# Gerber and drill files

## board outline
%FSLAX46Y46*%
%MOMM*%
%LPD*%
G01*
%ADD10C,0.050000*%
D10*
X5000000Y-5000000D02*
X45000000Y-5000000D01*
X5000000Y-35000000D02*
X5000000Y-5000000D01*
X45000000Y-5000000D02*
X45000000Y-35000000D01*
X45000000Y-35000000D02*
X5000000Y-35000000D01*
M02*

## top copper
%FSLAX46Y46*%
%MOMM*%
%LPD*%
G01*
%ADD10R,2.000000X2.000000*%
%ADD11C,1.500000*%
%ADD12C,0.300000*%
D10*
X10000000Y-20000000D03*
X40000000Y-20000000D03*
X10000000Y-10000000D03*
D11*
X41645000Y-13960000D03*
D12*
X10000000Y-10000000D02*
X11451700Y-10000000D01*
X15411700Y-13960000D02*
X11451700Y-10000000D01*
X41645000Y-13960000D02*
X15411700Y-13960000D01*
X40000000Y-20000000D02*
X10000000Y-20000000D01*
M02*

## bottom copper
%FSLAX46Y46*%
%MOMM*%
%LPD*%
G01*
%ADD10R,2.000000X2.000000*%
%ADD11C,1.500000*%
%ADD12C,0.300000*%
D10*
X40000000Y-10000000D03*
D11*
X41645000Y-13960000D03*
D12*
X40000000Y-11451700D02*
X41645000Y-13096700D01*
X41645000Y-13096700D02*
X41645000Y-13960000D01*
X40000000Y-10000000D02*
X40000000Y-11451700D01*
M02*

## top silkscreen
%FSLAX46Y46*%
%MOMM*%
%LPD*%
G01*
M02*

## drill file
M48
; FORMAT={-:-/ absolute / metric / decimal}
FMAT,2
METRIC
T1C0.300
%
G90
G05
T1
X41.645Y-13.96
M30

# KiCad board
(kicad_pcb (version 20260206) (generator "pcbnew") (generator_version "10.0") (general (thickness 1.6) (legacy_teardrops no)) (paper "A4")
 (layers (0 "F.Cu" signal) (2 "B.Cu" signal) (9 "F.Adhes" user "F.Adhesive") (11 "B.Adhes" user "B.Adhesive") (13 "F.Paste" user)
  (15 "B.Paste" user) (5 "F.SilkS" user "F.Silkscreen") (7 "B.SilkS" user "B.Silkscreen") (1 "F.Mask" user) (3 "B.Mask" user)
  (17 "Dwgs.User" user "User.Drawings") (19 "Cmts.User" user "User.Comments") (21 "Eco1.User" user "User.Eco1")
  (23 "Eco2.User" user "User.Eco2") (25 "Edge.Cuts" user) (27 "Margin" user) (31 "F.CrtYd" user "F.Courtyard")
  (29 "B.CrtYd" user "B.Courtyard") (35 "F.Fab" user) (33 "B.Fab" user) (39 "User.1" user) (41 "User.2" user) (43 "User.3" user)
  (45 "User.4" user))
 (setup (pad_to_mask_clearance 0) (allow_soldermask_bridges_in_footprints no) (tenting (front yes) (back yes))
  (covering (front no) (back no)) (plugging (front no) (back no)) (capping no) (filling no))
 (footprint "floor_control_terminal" (layer "F.Cu") (at 10 20)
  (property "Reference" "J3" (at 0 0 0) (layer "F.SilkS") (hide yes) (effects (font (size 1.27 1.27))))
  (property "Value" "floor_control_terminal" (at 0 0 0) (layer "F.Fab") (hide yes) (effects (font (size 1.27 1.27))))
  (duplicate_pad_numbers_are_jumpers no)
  (pad "1" smd rect (at 0 0) (size 2 2) (layers "F.Cu" "F.Mask" "F.Paste") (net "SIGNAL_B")))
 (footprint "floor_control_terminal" (layer "F.Cu") (at 40 20)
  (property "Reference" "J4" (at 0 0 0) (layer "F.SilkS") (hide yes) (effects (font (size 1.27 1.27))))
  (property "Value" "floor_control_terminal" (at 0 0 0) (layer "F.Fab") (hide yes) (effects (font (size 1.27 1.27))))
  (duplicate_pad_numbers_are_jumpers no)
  (pad "1" smd rect (at 0 0) (size 2 2) (layers "F.Cu" "F.Mask" "F.Paste") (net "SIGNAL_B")))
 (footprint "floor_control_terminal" (layer "F.Cu") (at 10 10)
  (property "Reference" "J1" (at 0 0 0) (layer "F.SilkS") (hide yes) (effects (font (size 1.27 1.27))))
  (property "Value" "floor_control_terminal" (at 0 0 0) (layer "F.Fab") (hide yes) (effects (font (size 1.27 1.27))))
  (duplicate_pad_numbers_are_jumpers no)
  (pad "1" smd rect (at 0 0) (size 2 2) (layers "F.Cu" "F.Mask" "F.Paste") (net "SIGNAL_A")))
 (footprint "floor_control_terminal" (layer "B.Cu") (at 40 10)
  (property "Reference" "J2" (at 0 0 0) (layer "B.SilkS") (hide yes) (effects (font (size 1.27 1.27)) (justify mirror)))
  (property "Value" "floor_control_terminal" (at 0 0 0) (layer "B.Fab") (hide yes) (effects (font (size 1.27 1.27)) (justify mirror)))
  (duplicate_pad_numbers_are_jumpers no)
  (pad "1" smd rect (at 0 0) (size 2 2) (layers "B.Cu" "B.Mask" "B.Paste") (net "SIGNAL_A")))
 (gr_line (start 5 5) (end 45 5) (stroke (width 0.05) (type default)) (layer "Edge.Cuts"))
 (gr_line (start 5 35) (end 5 5) (stroke (width 0.05) (type default)) (layer "Edge.Cuts"))
 (gr_line (start 45 5) (end 45 35) (stroke (width 0.05) (type default)) (layer "Edge.Cuts"))
 (gr_line (start 45 35) (end 5 35) (stroke (width 0.05) (type default)) (layer "Edge.Cuts"))
 (segment (start 10 10) (end 11.4517 10) (width 0.3) (layer "F.Cu") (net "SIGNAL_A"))
 (segment (start 15.4117 13.96) (end 11.4517 10) (width 0.3) (layer "F.Cu") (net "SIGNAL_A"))
 (segment (start 41.645 13.96) (end 15.4117 13.96) (width 0.3) (layer "F.Cu") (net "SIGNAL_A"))
 (via (at 41.645 13.96) (size 1.5) (drill 0.3) (layers "F.Cu" "B.Cu") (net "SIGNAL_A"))
 (segment (start 40 11.4517) (end 41.645 13.0967) (width 0.3) (layer "B.Cu") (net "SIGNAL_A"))
 (segment (start 41.645 13.0967) (end 41.645 13.96) (width 0.3) (layer "B.Cu") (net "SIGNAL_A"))
 (segment (start 40 10) (end 40 11.4517) (width 0.3) (layer "B.Cu") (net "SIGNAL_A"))
 (segment (start 40 20) (end 10 20) (width 0.3) (layer "F.Cu") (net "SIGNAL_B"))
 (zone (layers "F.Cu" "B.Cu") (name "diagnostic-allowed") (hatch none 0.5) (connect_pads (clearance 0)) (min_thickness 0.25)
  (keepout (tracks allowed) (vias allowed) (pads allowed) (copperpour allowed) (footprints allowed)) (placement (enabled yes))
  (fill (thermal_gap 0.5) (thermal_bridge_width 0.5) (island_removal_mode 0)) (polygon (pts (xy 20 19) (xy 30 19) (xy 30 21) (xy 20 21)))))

